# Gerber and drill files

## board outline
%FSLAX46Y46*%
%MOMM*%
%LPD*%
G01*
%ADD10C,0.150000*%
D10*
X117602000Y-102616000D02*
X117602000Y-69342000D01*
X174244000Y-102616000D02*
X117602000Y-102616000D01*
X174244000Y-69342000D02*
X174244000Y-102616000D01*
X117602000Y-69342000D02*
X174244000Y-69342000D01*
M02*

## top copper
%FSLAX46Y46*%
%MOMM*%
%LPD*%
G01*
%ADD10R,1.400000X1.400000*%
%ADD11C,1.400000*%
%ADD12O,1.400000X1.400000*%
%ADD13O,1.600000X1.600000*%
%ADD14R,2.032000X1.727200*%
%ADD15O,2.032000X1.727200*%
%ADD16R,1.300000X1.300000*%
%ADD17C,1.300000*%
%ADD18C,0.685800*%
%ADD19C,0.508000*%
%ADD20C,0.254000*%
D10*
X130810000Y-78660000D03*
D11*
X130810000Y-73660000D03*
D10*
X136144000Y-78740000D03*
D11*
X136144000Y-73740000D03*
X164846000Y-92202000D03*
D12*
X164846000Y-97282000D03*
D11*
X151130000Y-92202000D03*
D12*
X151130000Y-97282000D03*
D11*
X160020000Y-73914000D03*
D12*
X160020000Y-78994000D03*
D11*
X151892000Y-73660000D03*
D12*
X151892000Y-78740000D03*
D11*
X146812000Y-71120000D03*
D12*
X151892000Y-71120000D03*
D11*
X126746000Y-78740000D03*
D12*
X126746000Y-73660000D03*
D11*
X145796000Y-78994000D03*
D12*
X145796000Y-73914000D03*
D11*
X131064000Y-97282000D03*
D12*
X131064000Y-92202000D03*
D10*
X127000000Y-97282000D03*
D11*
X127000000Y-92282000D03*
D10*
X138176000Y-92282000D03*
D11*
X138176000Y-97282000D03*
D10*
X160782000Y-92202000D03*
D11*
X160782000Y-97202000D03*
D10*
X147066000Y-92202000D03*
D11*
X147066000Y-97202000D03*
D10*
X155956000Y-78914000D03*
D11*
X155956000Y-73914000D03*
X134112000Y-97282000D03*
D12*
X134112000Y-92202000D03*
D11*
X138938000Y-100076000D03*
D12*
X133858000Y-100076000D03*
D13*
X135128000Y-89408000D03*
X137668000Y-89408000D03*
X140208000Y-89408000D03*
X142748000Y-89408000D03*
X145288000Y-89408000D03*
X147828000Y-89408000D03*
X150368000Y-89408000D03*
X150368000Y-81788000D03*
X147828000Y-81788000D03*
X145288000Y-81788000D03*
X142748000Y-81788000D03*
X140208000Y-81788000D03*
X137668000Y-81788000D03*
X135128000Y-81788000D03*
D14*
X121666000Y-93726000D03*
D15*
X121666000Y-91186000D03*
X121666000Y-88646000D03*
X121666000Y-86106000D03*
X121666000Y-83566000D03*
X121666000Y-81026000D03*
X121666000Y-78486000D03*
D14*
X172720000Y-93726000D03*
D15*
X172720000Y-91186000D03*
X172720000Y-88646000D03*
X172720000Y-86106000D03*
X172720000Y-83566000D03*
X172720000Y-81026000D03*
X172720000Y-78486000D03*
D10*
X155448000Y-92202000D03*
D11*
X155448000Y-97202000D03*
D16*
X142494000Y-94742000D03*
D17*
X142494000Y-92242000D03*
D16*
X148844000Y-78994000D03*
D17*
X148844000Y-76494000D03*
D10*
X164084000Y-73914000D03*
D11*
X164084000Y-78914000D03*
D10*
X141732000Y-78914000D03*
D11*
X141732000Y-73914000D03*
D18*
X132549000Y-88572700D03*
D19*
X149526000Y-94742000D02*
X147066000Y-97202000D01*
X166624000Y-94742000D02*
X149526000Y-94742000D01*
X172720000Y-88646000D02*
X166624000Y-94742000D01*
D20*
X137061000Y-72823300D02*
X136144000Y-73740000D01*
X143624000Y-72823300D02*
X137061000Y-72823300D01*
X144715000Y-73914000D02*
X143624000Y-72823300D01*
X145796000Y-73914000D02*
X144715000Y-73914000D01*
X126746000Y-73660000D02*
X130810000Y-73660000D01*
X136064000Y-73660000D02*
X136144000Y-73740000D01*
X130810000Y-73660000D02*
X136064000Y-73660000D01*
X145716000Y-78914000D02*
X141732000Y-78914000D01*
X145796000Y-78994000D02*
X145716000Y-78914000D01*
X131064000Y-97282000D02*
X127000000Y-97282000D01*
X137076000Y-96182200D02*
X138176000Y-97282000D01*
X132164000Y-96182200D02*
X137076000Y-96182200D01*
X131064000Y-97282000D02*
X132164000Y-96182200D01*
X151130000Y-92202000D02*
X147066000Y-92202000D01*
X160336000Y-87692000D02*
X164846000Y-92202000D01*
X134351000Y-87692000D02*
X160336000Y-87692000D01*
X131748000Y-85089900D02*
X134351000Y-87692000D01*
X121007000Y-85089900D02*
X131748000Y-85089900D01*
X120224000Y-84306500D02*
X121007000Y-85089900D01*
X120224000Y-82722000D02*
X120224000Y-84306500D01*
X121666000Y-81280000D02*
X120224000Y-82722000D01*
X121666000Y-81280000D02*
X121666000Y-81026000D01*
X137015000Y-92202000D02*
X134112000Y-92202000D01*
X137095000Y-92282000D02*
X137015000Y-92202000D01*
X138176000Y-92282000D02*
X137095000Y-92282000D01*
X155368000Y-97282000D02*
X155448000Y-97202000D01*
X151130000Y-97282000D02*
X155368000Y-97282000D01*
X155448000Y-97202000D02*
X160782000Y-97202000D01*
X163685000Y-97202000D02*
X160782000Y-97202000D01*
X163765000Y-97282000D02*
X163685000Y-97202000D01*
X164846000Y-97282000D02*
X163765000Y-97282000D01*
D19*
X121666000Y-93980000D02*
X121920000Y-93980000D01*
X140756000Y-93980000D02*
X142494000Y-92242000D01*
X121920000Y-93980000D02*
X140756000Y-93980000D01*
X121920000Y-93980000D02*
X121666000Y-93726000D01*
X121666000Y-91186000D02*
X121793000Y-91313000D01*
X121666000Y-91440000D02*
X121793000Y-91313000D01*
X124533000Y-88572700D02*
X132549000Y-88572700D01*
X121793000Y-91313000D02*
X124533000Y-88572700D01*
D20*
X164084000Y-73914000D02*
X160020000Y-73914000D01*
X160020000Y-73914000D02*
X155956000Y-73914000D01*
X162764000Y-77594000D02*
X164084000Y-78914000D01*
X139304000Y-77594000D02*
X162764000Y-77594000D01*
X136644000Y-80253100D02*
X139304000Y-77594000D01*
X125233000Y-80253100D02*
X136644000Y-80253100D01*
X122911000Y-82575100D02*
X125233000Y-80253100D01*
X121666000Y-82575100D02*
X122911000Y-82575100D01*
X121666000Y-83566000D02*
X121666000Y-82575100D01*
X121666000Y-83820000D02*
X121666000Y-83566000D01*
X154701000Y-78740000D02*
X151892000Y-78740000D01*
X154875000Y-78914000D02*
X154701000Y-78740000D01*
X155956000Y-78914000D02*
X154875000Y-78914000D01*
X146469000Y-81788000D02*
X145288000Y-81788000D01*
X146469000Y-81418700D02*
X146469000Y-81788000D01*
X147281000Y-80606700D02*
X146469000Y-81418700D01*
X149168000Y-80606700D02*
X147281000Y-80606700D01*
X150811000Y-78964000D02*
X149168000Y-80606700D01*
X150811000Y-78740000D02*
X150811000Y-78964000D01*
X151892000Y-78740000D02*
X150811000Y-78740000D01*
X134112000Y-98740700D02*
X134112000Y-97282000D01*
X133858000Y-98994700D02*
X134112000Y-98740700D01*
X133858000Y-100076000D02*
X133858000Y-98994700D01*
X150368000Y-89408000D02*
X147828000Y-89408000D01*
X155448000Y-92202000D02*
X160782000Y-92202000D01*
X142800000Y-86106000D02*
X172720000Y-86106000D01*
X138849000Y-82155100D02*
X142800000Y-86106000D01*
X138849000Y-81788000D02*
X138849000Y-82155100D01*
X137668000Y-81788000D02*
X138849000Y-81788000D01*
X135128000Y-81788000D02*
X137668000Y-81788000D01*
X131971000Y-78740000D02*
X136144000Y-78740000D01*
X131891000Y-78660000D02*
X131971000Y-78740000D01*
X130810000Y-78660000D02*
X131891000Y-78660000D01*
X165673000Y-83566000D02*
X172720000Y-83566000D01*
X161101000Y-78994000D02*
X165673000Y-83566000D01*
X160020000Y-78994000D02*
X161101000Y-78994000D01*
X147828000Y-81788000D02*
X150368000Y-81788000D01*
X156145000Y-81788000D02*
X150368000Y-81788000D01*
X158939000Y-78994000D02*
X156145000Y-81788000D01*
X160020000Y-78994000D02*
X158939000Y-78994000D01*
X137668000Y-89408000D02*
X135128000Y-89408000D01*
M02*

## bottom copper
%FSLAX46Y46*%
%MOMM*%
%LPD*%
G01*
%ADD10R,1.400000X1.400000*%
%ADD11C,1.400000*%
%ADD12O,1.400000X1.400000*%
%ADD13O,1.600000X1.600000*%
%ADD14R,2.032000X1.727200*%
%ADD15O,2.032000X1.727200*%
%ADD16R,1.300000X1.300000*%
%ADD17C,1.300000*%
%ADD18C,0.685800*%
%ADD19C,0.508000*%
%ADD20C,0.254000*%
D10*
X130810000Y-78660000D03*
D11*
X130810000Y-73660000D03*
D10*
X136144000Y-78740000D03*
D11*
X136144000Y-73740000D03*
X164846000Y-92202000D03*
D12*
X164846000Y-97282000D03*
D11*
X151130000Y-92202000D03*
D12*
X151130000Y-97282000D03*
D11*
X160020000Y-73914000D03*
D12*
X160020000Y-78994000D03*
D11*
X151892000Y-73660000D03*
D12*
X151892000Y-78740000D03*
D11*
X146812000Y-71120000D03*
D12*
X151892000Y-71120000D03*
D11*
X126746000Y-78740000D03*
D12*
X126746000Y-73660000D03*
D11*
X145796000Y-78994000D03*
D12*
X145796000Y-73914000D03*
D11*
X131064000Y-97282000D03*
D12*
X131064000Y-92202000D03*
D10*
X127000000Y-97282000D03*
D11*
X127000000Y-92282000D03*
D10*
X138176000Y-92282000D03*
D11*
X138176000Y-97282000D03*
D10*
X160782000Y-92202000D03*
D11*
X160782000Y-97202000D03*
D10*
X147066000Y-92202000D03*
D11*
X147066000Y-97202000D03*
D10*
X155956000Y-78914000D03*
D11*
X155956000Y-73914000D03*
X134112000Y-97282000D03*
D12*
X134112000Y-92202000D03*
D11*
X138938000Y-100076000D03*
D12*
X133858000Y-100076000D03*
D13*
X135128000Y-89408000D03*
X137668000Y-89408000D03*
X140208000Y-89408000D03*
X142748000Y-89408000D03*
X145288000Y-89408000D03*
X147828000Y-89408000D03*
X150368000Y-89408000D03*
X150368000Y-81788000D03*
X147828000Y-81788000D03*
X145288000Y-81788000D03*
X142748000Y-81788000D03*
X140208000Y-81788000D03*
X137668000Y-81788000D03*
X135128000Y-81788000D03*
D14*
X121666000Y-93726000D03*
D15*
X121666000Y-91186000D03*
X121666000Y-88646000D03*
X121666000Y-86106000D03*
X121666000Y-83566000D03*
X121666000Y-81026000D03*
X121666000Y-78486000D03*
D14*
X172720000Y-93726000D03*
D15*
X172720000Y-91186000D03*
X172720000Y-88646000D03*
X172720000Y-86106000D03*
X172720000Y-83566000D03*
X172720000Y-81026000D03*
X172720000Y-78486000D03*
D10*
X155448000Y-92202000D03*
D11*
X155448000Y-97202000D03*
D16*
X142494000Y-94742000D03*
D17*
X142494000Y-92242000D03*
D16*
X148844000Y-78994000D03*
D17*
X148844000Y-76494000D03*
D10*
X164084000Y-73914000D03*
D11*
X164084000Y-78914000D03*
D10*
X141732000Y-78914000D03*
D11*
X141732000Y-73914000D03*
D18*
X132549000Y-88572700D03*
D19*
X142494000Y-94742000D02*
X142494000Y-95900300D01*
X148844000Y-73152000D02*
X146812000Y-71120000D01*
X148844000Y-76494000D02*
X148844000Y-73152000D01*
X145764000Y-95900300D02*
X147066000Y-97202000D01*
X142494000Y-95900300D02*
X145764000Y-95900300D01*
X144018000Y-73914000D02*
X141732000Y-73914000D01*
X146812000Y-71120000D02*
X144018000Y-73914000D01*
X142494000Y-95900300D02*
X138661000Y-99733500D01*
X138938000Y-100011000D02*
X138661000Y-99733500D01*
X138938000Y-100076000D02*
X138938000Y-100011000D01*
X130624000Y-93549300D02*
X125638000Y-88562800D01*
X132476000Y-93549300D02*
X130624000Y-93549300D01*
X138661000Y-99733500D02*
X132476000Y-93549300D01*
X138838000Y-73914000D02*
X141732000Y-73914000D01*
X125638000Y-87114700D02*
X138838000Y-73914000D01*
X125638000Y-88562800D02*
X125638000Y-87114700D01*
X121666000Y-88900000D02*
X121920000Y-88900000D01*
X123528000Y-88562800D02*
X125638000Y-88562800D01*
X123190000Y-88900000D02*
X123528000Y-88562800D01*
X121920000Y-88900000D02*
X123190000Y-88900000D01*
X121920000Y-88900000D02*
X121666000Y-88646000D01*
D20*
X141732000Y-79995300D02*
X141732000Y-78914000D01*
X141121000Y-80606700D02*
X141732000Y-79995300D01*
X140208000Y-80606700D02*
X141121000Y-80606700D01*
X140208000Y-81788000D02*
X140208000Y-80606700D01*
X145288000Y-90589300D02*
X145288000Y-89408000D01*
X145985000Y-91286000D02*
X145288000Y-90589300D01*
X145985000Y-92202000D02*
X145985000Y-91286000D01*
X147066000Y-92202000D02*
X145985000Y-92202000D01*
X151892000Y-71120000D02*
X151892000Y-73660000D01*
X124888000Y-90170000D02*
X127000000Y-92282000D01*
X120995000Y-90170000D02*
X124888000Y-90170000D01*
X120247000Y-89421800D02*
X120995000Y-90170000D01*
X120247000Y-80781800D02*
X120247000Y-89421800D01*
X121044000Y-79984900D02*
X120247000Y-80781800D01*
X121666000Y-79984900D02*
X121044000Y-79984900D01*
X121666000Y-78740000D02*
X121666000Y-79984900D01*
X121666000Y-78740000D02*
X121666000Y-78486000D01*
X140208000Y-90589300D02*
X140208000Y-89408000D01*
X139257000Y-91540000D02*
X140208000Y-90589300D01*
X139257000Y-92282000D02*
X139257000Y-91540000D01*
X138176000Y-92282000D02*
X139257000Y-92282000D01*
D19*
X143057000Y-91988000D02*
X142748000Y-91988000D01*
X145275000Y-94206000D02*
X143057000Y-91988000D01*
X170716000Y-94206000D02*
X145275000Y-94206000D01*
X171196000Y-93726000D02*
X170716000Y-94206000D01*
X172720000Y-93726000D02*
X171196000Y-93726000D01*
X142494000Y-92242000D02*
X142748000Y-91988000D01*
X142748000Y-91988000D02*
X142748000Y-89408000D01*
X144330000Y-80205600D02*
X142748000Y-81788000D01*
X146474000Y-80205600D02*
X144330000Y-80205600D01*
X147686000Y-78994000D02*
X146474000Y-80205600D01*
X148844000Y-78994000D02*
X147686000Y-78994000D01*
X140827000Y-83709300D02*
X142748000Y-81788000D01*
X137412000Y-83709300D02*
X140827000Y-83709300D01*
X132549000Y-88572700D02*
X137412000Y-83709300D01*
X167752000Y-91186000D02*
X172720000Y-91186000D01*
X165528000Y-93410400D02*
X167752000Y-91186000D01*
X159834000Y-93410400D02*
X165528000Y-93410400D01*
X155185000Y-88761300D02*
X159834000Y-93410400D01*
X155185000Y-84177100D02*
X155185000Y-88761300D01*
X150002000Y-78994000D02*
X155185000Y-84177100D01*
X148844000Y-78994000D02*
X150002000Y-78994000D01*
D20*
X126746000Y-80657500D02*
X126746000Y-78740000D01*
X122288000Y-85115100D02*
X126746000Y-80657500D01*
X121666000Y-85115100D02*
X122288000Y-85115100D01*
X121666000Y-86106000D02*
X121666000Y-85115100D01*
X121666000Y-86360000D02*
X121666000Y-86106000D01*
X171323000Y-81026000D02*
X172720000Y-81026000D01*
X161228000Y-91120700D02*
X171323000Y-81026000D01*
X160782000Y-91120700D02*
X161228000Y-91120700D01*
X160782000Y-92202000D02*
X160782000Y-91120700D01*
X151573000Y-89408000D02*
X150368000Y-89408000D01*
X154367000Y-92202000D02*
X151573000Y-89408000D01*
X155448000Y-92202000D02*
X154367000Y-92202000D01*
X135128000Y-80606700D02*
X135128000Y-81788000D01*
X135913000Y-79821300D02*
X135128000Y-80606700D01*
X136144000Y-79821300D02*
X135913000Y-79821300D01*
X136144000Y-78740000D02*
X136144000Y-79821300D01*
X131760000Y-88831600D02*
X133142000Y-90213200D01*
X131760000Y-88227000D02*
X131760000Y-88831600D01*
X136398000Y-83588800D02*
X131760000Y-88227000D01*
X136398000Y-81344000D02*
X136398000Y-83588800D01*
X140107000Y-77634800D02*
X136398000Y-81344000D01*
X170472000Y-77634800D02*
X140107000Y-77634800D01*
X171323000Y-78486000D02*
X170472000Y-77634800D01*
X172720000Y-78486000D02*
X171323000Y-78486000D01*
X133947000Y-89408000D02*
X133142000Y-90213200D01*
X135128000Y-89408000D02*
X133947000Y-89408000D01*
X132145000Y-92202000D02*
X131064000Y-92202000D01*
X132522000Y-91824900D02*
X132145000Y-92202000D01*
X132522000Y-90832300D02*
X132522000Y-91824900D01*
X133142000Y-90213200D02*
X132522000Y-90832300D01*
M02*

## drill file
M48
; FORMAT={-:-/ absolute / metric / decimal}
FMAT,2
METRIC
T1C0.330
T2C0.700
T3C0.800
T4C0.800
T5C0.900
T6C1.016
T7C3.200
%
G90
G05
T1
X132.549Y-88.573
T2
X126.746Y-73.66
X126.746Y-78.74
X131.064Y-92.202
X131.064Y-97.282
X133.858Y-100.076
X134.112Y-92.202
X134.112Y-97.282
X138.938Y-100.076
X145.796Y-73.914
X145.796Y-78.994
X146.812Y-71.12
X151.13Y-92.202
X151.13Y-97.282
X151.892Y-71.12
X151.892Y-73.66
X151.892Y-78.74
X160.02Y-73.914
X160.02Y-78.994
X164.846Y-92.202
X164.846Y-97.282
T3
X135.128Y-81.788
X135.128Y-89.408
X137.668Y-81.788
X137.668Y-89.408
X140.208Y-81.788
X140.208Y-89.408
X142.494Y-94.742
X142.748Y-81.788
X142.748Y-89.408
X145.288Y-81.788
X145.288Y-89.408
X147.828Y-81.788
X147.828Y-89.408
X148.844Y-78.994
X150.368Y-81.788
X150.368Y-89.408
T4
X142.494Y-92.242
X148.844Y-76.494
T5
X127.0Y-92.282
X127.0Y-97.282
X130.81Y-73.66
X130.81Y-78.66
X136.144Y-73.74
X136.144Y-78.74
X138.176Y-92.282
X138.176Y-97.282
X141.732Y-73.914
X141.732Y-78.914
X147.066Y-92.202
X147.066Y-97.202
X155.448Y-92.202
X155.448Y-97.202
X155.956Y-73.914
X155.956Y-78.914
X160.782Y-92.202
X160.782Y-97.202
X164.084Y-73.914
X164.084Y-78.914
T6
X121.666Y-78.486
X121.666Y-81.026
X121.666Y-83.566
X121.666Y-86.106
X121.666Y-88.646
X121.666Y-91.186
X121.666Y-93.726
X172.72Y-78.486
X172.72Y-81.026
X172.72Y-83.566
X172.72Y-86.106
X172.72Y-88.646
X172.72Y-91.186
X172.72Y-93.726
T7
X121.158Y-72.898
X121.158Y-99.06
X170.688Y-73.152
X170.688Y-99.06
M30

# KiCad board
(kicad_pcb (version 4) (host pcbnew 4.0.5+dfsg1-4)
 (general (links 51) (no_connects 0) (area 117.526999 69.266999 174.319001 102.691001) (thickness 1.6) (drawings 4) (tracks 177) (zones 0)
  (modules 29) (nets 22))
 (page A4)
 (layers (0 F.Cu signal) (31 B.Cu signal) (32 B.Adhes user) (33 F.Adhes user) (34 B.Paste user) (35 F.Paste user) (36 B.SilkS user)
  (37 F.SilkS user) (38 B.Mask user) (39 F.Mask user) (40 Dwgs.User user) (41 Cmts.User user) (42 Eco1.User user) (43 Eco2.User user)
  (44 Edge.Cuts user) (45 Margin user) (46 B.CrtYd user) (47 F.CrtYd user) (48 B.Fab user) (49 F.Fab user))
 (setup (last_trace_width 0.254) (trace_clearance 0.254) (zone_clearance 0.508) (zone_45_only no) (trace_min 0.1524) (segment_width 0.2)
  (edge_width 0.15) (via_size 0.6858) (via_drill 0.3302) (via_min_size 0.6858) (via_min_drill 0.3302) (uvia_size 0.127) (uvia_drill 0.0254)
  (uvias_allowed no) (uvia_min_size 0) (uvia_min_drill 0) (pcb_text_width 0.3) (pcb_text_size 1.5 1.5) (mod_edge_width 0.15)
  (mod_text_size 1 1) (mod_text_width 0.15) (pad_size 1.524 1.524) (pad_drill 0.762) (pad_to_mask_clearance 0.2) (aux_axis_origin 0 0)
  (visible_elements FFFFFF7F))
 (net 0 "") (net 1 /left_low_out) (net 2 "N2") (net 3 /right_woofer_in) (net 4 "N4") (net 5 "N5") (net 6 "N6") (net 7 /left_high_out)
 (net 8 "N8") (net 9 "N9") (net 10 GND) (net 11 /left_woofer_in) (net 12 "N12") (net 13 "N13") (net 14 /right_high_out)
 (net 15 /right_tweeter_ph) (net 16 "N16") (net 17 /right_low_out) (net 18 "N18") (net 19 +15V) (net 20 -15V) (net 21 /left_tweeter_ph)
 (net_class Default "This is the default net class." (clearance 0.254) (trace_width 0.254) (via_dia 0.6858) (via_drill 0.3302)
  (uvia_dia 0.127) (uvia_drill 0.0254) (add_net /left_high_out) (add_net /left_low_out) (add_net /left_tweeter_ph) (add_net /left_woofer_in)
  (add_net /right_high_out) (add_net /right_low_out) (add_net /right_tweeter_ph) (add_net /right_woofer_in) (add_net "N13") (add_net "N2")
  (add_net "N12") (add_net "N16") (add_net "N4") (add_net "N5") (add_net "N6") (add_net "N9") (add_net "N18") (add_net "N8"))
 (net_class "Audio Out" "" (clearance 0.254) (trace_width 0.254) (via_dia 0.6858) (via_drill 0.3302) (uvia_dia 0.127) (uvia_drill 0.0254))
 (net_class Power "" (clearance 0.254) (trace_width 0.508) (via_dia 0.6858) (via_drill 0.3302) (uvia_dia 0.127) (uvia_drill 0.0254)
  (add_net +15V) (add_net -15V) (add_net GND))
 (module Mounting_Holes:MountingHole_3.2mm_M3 (layer F.Cu) (at 121.158 99.06)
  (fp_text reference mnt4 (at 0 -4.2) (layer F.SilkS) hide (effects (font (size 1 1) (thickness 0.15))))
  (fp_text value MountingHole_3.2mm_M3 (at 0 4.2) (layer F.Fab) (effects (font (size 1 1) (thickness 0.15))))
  (pad 1 np_thru_hole circle (at 0 0) (size 3.2 3.2) (drill 3.2) (layers *.Cu *.Mask)))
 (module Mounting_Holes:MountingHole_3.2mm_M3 (layer F.Cu) (at 121.158 72.898)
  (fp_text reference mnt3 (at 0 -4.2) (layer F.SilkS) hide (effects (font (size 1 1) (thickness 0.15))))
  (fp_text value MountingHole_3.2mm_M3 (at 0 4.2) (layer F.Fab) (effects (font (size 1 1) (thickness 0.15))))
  (pad 1 np_thru_hole circle (at 0 0) (size 3.2 3.2) (drill 3.2) (layers *.Cu *.Mask)))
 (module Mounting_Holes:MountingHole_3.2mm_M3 (layer F.Cu) (at 170.688 99.06)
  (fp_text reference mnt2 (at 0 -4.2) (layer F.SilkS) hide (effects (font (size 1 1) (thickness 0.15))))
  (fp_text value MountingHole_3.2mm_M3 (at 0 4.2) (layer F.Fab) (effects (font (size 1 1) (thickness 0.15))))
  (pad 1 np_thru_hole circle (at 0 0) (size 3.2 3.2) (drill 3.2) (layers *.Cu *.Mask)))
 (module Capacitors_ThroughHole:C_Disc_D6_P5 (layer F.Cu) (at 130.81 78.66 90)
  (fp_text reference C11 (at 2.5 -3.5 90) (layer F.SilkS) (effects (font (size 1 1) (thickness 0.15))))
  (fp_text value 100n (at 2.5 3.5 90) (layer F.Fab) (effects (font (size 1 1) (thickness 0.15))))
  (pad 1 thru_hole rect (at 0 0 90) (size 1.4 1.4) (drill 0.9) (layers *.Cu *.Mask) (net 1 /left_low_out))
  (pad 2 thru_hole circle (at 5 0 90) (size 1.4 1.4) (drill 0.9) (layers *.Cu *.Mask) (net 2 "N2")))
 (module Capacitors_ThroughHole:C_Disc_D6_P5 (layer F.Cu) (at 136.144 78.74 90)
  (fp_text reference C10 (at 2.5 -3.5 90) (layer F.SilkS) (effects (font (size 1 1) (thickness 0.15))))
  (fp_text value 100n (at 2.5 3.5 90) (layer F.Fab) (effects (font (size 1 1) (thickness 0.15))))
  (pad 1 thru_hole rect (at 0 0 90) (size 1.4 1.4) (drill 0.9) (layers *.Cu *.Mask) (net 1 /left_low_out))
  (pad 2 thru_hole circle (at 5 0 90) (size 1.4 1.4) (drill 0.9) (layers *.Cu *.Mask) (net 2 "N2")))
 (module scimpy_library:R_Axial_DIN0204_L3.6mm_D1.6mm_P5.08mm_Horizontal (layer F.Cu) (at 164.846 92.202 270)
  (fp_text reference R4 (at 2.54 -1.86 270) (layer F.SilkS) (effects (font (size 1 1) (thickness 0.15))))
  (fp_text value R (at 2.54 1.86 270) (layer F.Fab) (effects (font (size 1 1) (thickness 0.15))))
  (pad 1 thru_hole circle (at 0 0 270) (size 1.4 1.4) (drill 0.7) (layers *.Cu *.Mask) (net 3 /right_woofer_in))
  (pad 2 thru_hole oval (at 5.08 0 270) (size 1.4 1.4) (drill 0.7) (layers *.Cu *.Mask) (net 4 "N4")))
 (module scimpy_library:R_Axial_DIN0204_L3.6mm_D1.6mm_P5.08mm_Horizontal (layer F.Cu) (at 151.13 92.202 270)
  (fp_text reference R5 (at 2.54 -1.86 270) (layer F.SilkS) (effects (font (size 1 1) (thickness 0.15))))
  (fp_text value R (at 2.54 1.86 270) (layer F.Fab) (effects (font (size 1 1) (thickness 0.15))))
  (pad 1 thru_hole circle (at 0 0 270) (size 1.4 1.4) (drill 0.7) (layers *.Cu *.Mask) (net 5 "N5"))
  (pad 2 thru_hole oval (at 5.08 0 270) (size 1.4 1.4) (drill 0.7) (layers *.Cu *.Mask) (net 4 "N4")))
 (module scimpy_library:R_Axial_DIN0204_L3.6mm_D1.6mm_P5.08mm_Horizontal (layer F.Cu) (at 160.02 73.914 270)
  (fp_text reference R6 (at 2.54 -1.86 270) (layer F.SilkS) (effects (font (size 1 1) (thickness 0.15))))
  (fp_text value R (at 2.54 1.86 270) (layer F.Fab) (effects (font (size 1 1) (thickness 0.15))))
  (pad 1 thru_hole circle (at 0 0 270) (size 1.4 1.4) (drill 0.7) (layers *.Cu *.Mask) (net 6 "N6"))
  (pad 2 thru_hole oval (at 5.08 0 270) (size 1.4 1.4) (drill 0.7) (layers *.Cu *.Mask) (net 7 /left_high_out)))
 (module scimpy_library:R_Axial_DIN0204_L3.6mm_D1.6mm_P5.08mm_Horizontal (layer F.Cu) (at 151.892 73.66 270)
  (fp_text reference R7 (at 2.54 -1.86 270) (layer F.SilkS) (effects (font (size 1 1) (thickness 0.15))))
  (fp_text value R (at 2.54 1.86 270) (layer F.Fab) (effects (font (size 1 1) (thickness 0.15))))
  (pad 1 thru_hole circle (at 0 0 270) (size 1.4 1.4) (drill 0.7) (layers *.Cu *.Mask) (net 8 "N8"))
  (pad 2 thru_hole oval (at 5.08 0 270) (size 1.4 1.4) (drill 0.7) (layers *.Cu *.Mask) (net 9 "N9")))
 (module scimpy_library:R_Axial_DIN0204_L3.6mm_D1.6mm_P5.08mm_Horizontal (layer F.Cu) (at 146.812 71.12)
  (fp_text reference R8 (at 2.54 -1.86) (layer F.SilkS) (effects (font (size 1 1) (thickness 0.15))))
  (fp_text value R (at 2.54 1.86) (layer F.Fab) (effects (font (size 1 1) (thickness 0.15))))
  (pad 1 thru_hole circle (at 0 0) (size 1.4 1.4) (drill 0.7) (layers *.Cu *.Mask) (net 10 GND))
  (pad 2 thru_hole oval (at 5.08 0) (size 1.4 1.4) (drill 0.7) (layers *.Cu *.Mask) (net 8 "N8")))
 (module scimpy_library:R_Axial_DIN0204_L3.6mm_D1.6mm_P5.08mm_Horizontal (layer F.Cu) (at 126.746 78.74 90)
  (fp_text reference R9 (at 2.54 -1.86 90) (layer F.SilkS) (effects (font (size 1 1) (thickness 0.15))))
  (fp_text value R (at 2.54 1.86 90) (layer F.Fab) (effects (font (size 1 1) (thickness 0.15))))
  (pad 1 thru_hole circle (at 0 0 90) (size 1.4 1.4) (drill 0.7) (layers *.Cu *.Mask) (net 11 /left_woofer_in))
  (pad 2 thru_hole oval (at 5.08 0 90) (size 1.4 1.4) (drill 0.7) (layers *.Cu *.Mask) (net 2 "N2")))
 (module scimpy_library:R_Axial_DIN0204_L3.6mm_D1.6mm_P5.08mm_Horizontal (layer F.Cu) (at 145.796 78.994 90)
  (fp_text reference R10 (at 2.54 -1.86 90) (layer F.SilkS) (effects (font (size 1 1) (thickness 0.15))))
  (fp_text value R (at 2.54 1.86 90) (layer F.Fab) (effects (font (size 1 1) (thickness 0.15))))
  (pad 1 thru_hole circle (at 0 0 90) (size 1.4 1.4) (drill 0.7) (layers *.Cu *.Mask) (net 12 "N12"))
  (pad 2 thru_hole oval (at 5.08 0 90) (size 1.4 1.4) (drill 0.7) (layers *.Cu *.Mask) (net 2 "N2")))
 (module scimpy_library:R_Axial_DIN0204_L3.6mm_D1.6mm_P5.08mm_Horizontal (layer F.Cu) (at 131.064 97.282 90)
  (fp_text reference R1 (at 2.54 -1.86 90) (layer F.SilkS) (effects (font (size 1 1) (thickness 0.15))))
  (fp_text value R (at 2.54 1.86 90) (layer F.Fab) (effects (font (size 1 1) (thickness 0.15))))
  (pad 1 thru_hole circle (at 0 0 90) (size 1.4 1.4) (drill 0.7) (layers *.Cu *.Mask) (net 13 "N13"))
  (pad 2 thru_hole oval (at 5.08 0 90) (size 1.4 1.4) (drill 0.7) (layers *.Cu *.Mask) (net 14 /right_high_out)))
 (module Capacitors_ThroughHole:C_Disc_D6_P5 (layer F.Cu) (at 127 97.282 90)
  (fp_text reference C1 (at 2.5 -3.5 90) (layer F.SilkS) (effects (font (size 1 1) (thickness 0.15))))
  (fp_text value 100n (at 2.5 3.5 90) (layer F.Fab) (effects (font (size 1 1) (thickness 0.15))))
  (pad 1 thru_hole rect (at 0 0 90) (size 1.4 1.4) (drill 0.9) (layers *.Cu *.Mask) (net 13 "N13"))
  (pad 2 thru_hole circle (at 5 0 90) (size 1.4 1.4) (drill 0.9) (layers *.Cu *.Mask) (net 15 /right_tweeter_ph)))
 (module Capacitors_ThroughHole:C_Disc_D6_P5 (layer F.Cu) (at 138.176 92.282 270)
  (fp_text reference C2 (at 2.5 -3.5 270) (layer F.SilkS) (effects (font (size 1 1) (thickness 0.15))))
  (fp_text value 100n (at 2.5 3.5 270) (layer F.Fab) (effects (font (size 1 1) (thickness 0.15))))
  (pad 1 thru_hole rect (at 0 0 270) (size 1.4 1.4) (drill 0.9) (layers *.Cu *.Mask) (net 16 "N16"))
  (pad 2 thru_hole circle (at 5 0 270) (size 1.4 1.4) (drill 0.9) (layers *.Cu *.Mask) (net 13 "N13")))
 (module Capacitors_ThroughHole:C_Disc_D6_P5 (layer F.Cu) (at 160.782 92.202 270)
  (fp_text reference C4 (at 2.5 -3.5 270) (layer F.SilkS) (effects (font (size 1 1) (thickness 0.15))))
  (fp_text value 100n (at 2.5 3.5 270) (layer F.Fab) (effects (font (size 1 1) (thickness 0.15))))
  (pad 1 thru_hole rect (at 0 0 270) (size 1.4 1.4) (drill 0.9) (layers *.Cu *.Mask) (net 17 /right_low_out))
  (pad 2 thru_hole circle (at 5 0 270) (size 1.4 1.4) (drill 0.9) (layers *.Cu *.Mask) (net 4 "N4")))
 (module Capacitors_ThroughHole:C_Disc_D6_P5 (layer F.Cu) (at 147.066 92.202 270)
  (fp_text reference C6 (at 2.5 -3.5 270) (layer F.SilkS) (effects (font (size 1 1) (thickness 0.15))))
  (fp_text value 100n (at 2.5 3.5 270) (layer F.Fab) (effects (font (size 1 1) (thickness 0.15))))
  (pad 1 thru_hole rect (at 0 0 270) (size 1.4 1.4) (drill 0.9) (layers *.Cu *.Mask) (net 5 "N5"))
  (pad 2 thru_hole circle (at 5 0 270) (size 1.4 1.4) (drill 0.9) (layers *.Cu *.Mask) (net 10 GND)))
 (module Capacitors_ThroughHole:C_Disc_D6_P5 (layer F.Cu) (at 155.956 78.914 90)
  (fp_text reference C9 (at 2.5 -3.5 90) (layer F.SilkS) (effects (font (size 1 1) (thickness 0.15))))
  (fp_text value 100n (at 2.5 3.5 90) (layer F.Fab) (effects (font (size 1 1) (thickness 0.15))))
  (pad 1 thru_hole rect (at 0 0 90) (size 1.4 1.4) (drill 0.9) (layers *.Cu *.Mask) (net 9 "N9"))
  (pad 2 thru_hole circle (at 5 0 90) (size 1.4 1.4) (drill 0.9) (layers *.Cu *.Mask) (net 6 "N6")))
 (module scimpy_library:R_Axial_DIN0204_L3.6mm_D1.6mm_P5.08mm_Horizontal (layer F.Cu) (at 134.112 97.282 90)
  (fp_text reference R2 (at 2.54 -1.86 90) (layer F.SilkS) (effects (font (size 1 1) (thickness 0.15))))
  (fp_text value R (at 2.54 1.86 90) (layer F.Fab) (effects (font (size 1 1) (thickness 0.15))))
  (pad 1 thru_hole circle (at 0 0 90) (size 1.4 1.4) (drill 0.7) (layers *.Cu *.Mask) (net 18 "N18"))
  (pad 2 thru_hole oval (at 5.08 0 90) (size 1.4 1.4) (drill 0.7) (layers *.Cu *.Mask) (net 16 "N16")))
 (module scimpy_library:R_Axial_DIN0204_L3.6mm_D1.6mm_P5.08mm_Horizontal (layer F.Cu) (at 138.938 100.076 180)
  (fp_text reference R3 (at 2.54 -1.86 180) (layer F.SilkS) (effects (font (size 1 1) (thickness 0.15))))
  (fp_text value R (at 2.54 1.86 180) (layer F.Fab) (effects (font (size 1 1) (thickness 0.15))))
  (pad 1 thru_hole circle (at 0 0 180) (size 1.4 1.4) (drill 0.7) (layers *.Cu *.Mask) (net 10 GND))
  (pad 2 thru_hole oval (at 5.08 0 180) (size 1.4 1.4) (drill 0.7) (layers *.Cu *.Mask) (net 18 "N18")))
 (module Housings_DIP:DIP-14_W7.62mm (layer F.Cu) (at 135.128 89.408 90)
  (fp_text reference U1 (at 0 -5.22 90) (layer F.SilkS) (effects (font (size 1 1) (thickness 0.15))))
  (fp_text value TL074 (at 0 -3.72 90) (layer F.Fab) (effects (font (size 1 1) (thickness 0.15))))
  (pad 1 thru_hole oval (at 0 0 90) (size 1.6 1.6) (drill 0.8) (layers *.Cu *.Mask) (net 14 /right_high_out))
  (pad 2 thru_hole oval (at 0 2.54 90) (size 1.6 1.6) (drill 0.8) (layers *.Cu *.Mask) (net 14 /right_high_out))
  (pad 3 thru_hole oval (at 0 5.08 90) (size 1.6 1.6) (drill 0.8) (layers *.Cu *.Mask) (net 16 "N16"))
  (pad 4 thru_hole oval (at 0 7.62 90) (size 1.6 1.6) (drill 0.8) (layers *.Cu *.Mask) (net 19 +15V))
  (pad 5 thru_hole oval (at 0 10.16 90) (size 1.6 1.6) (drill 0.8) (layers *.Cu *.Mask) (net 5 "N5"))
  (pad 6 thru_hole oval (at 0 12.7 90) (size 1.6 1.6) (drill 0.8) (layers *.Cu *.Mask) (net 17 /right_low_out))
  (pad 7 thru_hole oval (at 0 15.24 90) (size 1.6 1.6) (drill 0.8) (layers *.Cu *.Mask) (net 17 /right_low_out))
  (pad 8 thru_hole oval (at 7.62 15.24 90) (size 1.6 1.6) (drill 0.8) (layers *.Cu *.Mask) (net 7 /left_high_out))
  (pad 9 thru_hole oval (at 7.62 12.7 90) (size 1.6 1.6) (drill 0.8) (layers *.Cu *.Mask) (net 7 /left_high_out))
  (pad 10 thru_hole oval (at 7.62 10.16 90) (size 1.6 1.6) (drill 0.8) (layers *.Cu *.Mask) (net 9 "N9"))
  (pad 11 thru_hole oval (at 7.62 7.62 90) (size 1.6 1.6) (drill 0.8) (layers *.Cu *.Mask) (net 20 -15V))
  (pad 12 thru_hole oval (at 7.62 5.08 90) (size 1.6 1.6) (drill 0.8) (layers *.Cu *.Mask) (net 12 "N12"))
  (pad 13 thru_hole oval (at 7.62 2.54 90) (size 1.6 1.6) (drill 0.8) (layers *.Cu *.Mask) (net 1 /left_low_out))
  (pad 14 thru_hole oval (at 7.62 0 90) (size 1.6 1.6) (drill 0.8) (layers *.Cu *.Mask) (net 1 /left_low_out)))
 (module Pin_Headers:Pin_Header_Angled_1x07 (layer F.Cu) (at 121.666 93.726 180)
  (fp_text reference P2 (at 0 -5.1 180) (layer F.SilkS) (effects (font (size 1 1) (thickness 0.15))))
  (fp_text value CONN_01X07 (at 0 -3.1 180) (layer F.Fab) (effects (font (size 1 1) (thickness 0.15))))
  (pad 1 thru_hole rect (at 0 0 180) (size 2.032 1.7272) (drill 1.016) (layers *.Cu *.Mask) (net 19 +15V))
  (pad 2 thru_hole oval (at 0 2.54 180) (size 2.032 1.7272) (drill 1.016) (layers *.Cu *.Mask) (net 20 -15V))
  (pad 3 thru_hole oval (at 0 5.08 180) (size 2.032 1.7272) (drill 1.016) (layers *.Cu *.Mask) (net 10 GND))
  (pad 4 thru_hole oval (at 0 7.62 180) (size 2.032 1.7272) (drill 1.016) (layers *.Cu *.Mask) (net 11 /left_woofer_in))
  (pad 5 thru_hole oval (at 0 10.16 180) (size 2.032 1.7272) (drill 1.016) (layers *.Cu *.Mask) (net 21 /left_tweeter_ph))
  (pad 6 thru_hole oval (at 0 12.7 180) (size 2.032 1.7272) (drill 1.016) (layers *.Cu *.Mask) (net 3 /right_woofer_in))
  (pad 7 thru_hole oval (at 0 15.24 180) (size 2.032 1.7272) (drill 1.016) (layers *.Cu *.Mask) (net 15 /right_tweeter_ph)))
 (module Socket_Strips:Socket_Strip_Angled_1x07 (layer F.Cu) (at 172.72 93.726 90)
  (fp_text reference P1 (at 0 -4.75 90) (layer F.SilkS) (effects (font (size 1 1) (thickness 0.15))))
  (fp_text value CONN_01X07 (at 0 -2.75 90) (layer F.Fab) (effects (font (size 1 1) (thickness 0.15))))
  (pad 1 thru_hole rect (at 0 0 90) (size 1.7272 2.032) (drill 1.016) (layers *.Cu *.Mask) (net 19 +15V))
  (pad 2 thru_hole oval (at 2.54 0 90) (size 1.7272 2.032) (drill 1.016) (layers *.Cu *.Mask) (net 20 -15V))
  (pad 3 thru_hole oval (at 5.08 0 90) (size 1.7272 2.032) (drill 1.016) (layers *.Cu *.Mask) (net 10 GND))
  (pad 4 thru_hole oval (at 7.62 0 90) (size 1.7272 2.032) (drill 1.016) (layers *.Cu *.Mask) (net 1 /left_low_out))
  (pad 5 thru_hole oval (at 10.16 0 90) (size 1.7272 2.032) (drill 1.016) (layers *.Cu *.Mask) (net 7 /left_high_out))
  (pad 6 thru_hole oval (at 12.7 0 90) (size 1.7272 2.032) (drill 1.016) (layers *.Cu *.Mask) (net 17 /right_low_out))
  (pad 7 thru_hole oval (at 15.24 0 90) (size 1.7272 2.032) (drill 1.016) (layers *.Cu *.Mask) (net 14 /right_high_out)))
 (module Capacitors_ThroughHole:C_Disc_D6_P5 (layer F.Cu) (at 155.448 92.202 270)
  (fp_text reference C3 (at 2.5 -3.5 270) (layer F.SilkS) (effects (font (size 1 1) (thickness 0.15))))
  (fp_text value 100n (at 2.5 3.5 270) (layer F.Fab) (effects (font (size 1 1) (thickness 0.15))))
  (pad 1 thru_hole rect (at 0 0 270) (size 1.4 1.4) (drill 0.9) (layers *.Cu *.Mask) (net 17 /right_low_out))
  (pad 2 thru_hole circle (at 5 0 270) (size 1.4 1.4) (drill 0.9) (layers *.Cu *.Mask) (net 4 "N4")))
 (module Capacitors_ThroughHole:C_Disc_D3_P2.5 (layer F.Cu) (at 142.494 94.742 90)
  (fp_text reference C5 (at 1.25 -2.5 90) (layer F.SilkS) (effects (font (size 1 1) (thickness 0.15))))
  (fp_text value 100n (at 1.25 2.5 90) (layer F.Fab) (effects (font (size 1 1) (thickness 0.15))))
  (pad 1 thru_hole rect (at 0 0 90) (size 1.3 1.3) (drill 0.8) (layers *.Cu *.Mask) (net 10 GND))
  (pad 2 thru_hole circle (at 2.5 0 90) (size 1.3 1.3) (drill 0.8001) (layers *.Cu *.Mask) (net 19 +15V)))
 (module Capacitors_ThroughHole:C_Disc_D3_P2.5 (layer F.Cu) (at 148.844 78.994 90)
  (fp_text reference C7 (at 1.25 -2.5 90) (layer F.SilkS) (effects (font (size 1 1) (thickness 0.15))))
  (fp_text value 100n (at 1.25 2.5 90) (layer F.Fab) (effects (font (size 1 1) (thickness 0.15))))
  (pad 1 thru_hole rect (at 0 0 90) (size 1.3 1.3) (drill 0.8) (layers *.Cu *.Mask) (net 20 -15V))
  (pad 2 thru_hole circle (at 2.5 0 90) (size 1.3 1.3) (drill 0.8001) (layers *.Cu *.Mask) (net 10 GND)))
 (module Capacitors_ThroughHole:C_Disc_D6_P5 (layer F.Cu) (at 164.084 73.914 270)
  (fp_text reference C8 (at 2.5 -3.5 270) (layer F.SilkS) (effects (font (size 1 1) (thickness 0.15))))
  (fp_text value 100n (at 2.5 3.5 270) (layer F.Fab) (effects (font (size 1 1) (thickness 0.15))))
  (pad 1 thru_hole rect (at 0 0 270) (size 1.4 1.4) (drill 0.9) (layers *.Cu *.Mask) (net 6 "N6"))
  (pad 2 thru_hole circle (at 5 0 270) (size 1.4 1.4) (drill 0.9) (layers *.Cu *.Mask) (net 21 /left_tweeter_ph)))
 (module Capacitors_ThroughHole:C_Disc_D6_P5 (layer F.Cu) (at 141.732 78.914 90)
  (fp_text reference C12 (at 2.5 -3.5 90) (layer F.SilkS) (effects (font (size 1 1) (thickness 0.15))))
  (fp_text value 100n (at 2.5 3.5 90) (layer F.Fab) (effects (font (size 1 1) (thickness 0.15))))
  (pad 1 thru_hole rect (at 0 0 90) (size 1.4 1.4) (drill 0.9) (layers *.Cu *.Mask) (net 12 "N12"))
  (pad 2 thru_hole circle (at 5 0 90) (size 1.4 1.4) (drill 0.9) (layers *.Cu *.Mask) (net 10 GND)))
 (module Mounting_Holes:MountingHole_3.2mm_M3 (layer F.Cu) (at 170.688 73.152)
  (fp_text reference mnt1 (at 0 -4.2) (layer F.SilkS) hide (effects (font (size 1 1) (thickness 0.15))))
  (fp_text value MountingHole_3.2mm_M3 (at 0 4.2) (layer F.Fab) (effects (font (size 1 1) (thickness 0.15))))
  (pad 1 np_thru_hole circle (at 0 0) (size 3.2 3.2) (drill 3.2) (layers *.Cu *.Mask)))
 (gr_line (start 117.602 102.616) (end 117.602 69.342) (angle 90) (layer Edge.Cuts) (width 0.15))
 (gr_line (start 174.244 102.616) (end 117.602 102.616) (angle 90) (layer Edge.Cuts) (width 0.15))
 (gr_line (start 174.244 69.342) (end 174.244 102.616) (angle 90) (layer Edge.Cuts) (width 0.15))
 (gr_line (start 117.602 69.342) (end 174.244 69.342) (angle 90) (layer Edge.Cuts) (width 0.15))
 (segment (start 149.526 94.742) (end 147.066 97.202) (width 0.508) (layer F.Cu) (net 10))
 (segment (start 166.624 94.742) (end 149.526 94.742) (width 0.508) (layer F.Cu) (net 10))
 (segment (start 172.72 88.646) (end 166.624 94.742) (width 0.508) (layer F.Cu) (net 10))
 (segment (start 142.494 94.742) (end 142.494 95.9003) (width 0.508) (layer B.Cu) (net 10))
 (segment (start 148.844 73.152) (end 146.812 71.12) (width 0.508) (layer B.Cu) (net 10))
 (segment (start 148.844 76.494) (end 148.844 73.152) (width 0.508) (layer B.Cu) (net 10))
 (segment (start 145.764 95.9003) (end 147.066 97.202) (width 0.508) (layer B.Cu) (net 10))
 (segment (start 142.494 95.9003) (end 145.764 95.9003) (width 0.508) (layer B.Cu) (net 10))
 (segment (start 144.018 73.914) (end 141.732 73.914) (width 0.508) (layer B.Cu) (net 10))
 (segment (start 146.812 71.12) (end 144.018 73.914) (width 0.508) (layer B.Cu) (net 10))
 (segment (start 142.494 95.9003) (end 138.661 99.7335) (width 0.508) (layer B.Cu) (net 10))
 (segment (start 138.938 100.011) (end 138.661 99.7335) (width 0.508) (layer B.Cu) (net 10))
 (segment (start 138.938 100.076) (end 138.938 100.011) (width 0.508) (layer B.Cu) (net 10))
 (segment (start 130.624 93.5493) (end 125.638 88.5628) (width 0.508) (layer B.Cu) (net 10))
 (segment (start 132.476 93.5493) (end 130.624 93.5493) (width 0.508) (layer B.Cu) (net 10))
 (segment (start 138.661 99.7335) (end 132.476 93.5493) (width 0.508) (layer B.Cu) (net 10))
 (segment (start 138.838 73.914) (end 141.732 73.914) (width 0.508) (layer B.Cu) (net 10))
 (segment (start 125.638 87.1147) (end 138.838 73.914) (width 0.508) (layer B.Cu) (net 10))
 (segment (start 125.638 88.5628) (end 125.638 87.1147) (width 0.508) (layer B.Cu) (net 10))
 (segment (start 121.666 88.9) (end 121.92 88.9) (width 0.508) (layer B.Cu) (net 10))
 (segment (start 123.528 88.5628) (end 125.638 88.5628) (width 0.508) (layer B.Cu) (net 10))
 (segment (start 123.19 88.9) (end 123.528 88.5628) (width 0.508) (layer B.Cu) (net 10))
 (segment (start 121.92 88.9) (end 123.19 88.9) (width 0.508) (layer B.Cu) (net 10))
 (segment (start 121.92 88.9) (end 121.666 88.646) (width 0.508) (layer B.Cu) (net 10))
 (segment (start 137.061 72.8233) (end 136.144 73.74) (width 0.254) (layer F.Cu) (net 2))
 (segment (start 143.624 72.8233) (end 137.061 72.8233) (width 0.254) (layer F.Cu) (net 2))
 (segment (start 144.715 73.914) (end 143.624 72.8233) (width 0.254) (layer F.Cu) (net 2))
 (segment (start 145.796 73.914) (end 144.715 73.914) (width 0.254) (layer F.Cu) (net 2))
 (segment (start 126.746 73.66) (end 130.81 73.66) (width 0.254) (layer F.Cu) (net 2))
 (segment (start 136.064 73.66) (end 136.144 73.74) (width 0.254) (layer F.Cu) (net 2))
 (segment (start 130.81 73.66) (end 136.064 73.66) (width 0.254) (layer F.Cu) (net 2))
 (segment (start 141.732 79.9953) (end 141.732 78.914) (width 0.254) (layer B.Cu) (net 12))
 (segment (start 141.121 80.6067) (end 141.732 79.9953) (width 0.254) (layer B.Cu) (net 12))
 (segment (start 140.208 80.6067) (end 141.121 80.6067) (width 0.254) (layer B.Cu) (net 12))
 (segment (start 140.208 81.788) (end 140.208 80.6067) (width 0.254) (layer B.Cu) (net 12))
 (segment (start 145.716 78.914) (end 141.732 78.914) (width 0.254) (layer F.Cu) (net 12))
 (segment (start 145.796 78.994) (end 145.716 78.914) (width 0.254) (layer F.Cu) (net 12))
 (segment (start 131.064 97.282) (end 127 97.282) (width 0.254) (layer F.Cu) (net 13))
 (segment (start 137.076 96.1822) (end 138.176 97.282) (width 0.254) (layer F.Cu) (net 13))
 (segment (start 132.164 96.1822) (end 137.076 96.1822) (width 0.254) (layer F.Cu) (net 13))
 (segment (start 131.064 97.282) (end 132.164 96.1822) (width 0.254) (layer F.Cu) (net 13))
 (segment (start 151.13 92.202) (end 147.066 92.202) (width 0.254) (layer F.Cu) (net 5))
 (segment (start 145.288 90.5893) (end 145.288 89.408) (width 0.254) (layer B.Cu) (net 5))
 (segment (start 145.985 91.286) (end 145.288 90.5893) (width 0.254) (layer B.Cu) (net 5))
 (segment (start 145.985 92.202) (end 145.985 91.286) (width 0.254) (layer B.Cu) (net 5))
 (segment (start 147.066 92.202) (end 145.985 92.202) (width 0.254) (layer B.Cu) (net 5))
 (segment (start 151.892 71.12) (end 151.892 73.66) (width 0.254) (layer B.Cu) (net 8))
 (segment (start 124.888 90.17) (end 127 92.282) (width 0.254) (layer B.Cu) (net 15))
 (segment (start 120.995 90.17) (end 124.888 90.17) (width 0.254) (layer B.Cu) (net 15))
 (segment (start 120.247 89.4218) (end 120.995 90.17) (width 0.254) (layer B.Cu) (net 15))
 (segment (start 120.247 80.7818) (end 120.247 89.4218) (width 0.254) (layer B.Cu) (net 15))
 (segment (start 121.044 79.9849) (end 120.247 80.7818) (width 0.254) (layer B.Cu) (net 15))
 (segment (start 121.666 79.9849) (end 121.044 79.9849) (width 0.254) (layer B.Cu) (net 15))
 (segment (start 121.666 78.74) (end 121.666 79.9849) (width 0.254) (layer B.Cu) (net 15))
 (segment (start 121.666 78.74) (end 121.666 78.486) (width 0.254) (layer B.Cu) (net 15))
 (segment (start 160.336 87.692) (end 164.846 92.202) (width 0.254) (layer F.Cu) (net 3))
 (segment (start 134.351 87.692) (end 160.336 87.692) (width 0.254) (layer F.Cu) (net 3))
 (segment (start 131.748 85.0899) (end 134.351 87.692) (width 0.254) (layer F.Cu) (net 3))
 (segment (start 121.007 85.0899) (end 131.748 85.0899) (width 0.254) (layer F.Cu) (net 3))
 (segment (start 120.224 84.3065) (end 121.007 85.0899) (width 0.254) (layer F.Cu) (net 3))
 (segment (start 120.224 82.722) (end 120.224 84.3065) (width 0.254) (layer F.Cu) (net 3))
 (segment (start 121.666 81.28) (end 120.224 82.722) (width 0.254) (layer F.Cu) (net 3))
 (segment (start 121.666 81.28) (end 121.666 81.026) (width 0.254) (layer F.Cu) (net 3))
 (segment (start 140.208 90.5893) (end 140.208 89.408) (width 0.254) (layer B.Cu) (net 16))
 (segment (start 139.257 91.54) (end 140.208 90.5893) (width 0.254) (layer B.Cu) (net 16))
 (segment (start 139.257 92.282) (end 139.257 91.54) (width 0.254) (layer B.Cu) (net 16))
 (segment (start 138.176 92.282) (end 139.257 92.282) (width 0.254) (layer B.Cu) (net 16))
 (segment (start 137.015 92.202) (end 134.112 92.202) (width 0.254) (layer F.Cu) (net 16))
 (segment (start 137.095 92.282) (end 137.015 92.202) (width 0.254) (layer F.Cu) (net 16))
 (segment (start 138.176 92.282) (end 137.095 92.282) (width 0.254) (layer F.Cu) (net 16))
 (segment (start 155.368 97.282) (end 155.448 97.202) (width 0.254) (layer F.Cu) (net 4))
 (segment (start 151.13 97.282) (end 155.368 97.282) (width 0.254) (layer F.Cu) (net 4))
 (segment (start 155.448 97.202) (end 160.782 97.202) (width 0.254) (layer F.Cu) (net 4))
 (segment (start 163.685 97.202) (end 160.782 97.202) (width 0.254) (layer F.Cu) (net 4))
 (segment (start 163.765 97.282) (end 163.685 97.202) (width 0.254) (layer F.Cu) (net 4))
 (segment (start 164.846 97.282) (end 163.765 97.282) (width 0.254) (layer F.Cu) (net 4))
 (segment (start 143.057 91.988) (end 142.748 91.988) (width 0.508) (layer B.Cu) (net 19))
 (segment (start 145.275 94.206) (end 143.057 91.988) (width 0.508) (layer B.Cu) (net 19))
 (segment (start 170.716 94.206) (end 145.275 94.206) (width 0.508) (layer B.Cu) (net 19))
 (segment (start 171.196 93.726) (end 170.716 94.206) (width 0.508) (layer B.Cu) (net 19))
 (segment (start 172.72 93.726) (end 171.196 93.726) (width 0.508) (layer B.Cu) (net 19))
 (segment (start 142.494 92.242) (end 142.748 91.988) (width 0.508) (layer B.Cu) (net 19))
 (segment (start 142.748 91.988) (end 142.748 89.408) (width 0.508) (layer B.Cu) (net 19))
 (segment (start 121.666 93.98) (end 121.92 93.98) (width 0.508) (layer F.Cu) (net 19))
 (segment (start 140.756 93.98) (end 142.494 92.242) (width 0.508) (layer F.Cu) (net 19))
 (segment (start 121.92 93.98) (end 140.756 93.98) (width 0.508) (layer F.Cu) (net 19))
 (segment (start 121.92 93.98) (end 121.666 93.726) (width 0.508) (layer F.Cu) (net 19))
 (via (at 132.549 88.5727) (size 0.6858) (layers F.Cu B.Cu) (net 20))
 (segment (start 144.33 80.2056) (end 142.748 81.788) (width 0.508) (layer B.Cu) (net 20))
 (segment (start 146.474 80.2056) (end 144.33 80.2056) (width 0.508) (layer B.Cu) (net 20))
 (segment (start 147.686 78.994) (end 146.474 80.2056) (width 0.508) (layer B.Cu) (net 20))
 (segment (start 148.844 78.994) (end 147.686 78.994) (width 0.508) (layer B.Cu) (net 20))
 (segment (start 140.827 83.7093) (end 142.748 81.788) (width 0.508) (layer B.Cu) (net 20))
 (segment (start 137.412 83.7093) (end 140.827 83.7093) (width 0.508) (layer B.Cu) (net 20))
 (segment (start 132.549 88.5727) (end 137.412 83.7093) (width 0.508) (layer B.Cu) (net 20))
 (segment (start 167.752 91.186) (end 172.72 91.186) (width 0.508) (layer B.Cu) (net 20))
 (segment (start 165.528 93.4104) (end 167.752 91.186) (width 0.508) (layer B.Cu) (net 20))
 (segment (start 159.834 93.4104) (end 165.528 93.4104) (width 0.508) (layer B.Cu) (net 20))
 (segment (start 155.185 88.7613) (end 159.834 93.4104) (width 0.508) (layer B.Cu) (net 20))
 (segment (start 155.185 84.1771) (end 155.185 88.7613) (width 0.508) (layer B.Cu) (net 20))
 (segment (start 150.002 78.994) (end 155.185 84.1771) (width 0.508) (layer B.Cu) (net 20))
 (segment (start 148.844 78.994) (end 150.002 78.994) (width 0.508) (layer B.Cu) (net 20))
 (segment (start 121.666 91.186) (end 121.793 91.313) (width 0.508) (layer F.Cu) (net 20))
 (segment (start 121.666 91.44) (end 121.793 91.313) (width 0.508) (layer F.Cu) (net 20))
 (segment (start 124.533 88.5727) (end 132.549 88.5727) (width 0.508) (layer F.Cu) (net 20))
 (segment (start 121.793 91.313) (end 124.533 88.5727) (width 0.508) (layer F.Cu) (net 20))
 (segment (start 164.084 73.914) (end 160.02 73.914) (width 0.254) (layer F.Cu) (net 6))
 (segment (start 160.02 73.914) (end 155.956 73.914) (width 0.254) (layer F.Cu) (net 6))
 (segment (start 162.764 77.594) (end 164.084 78.914) (width 0.254) (layer F.Cu) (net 21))
 (segment (start 139.304 77.594) (end 162.764 77.594) (width 0.254) (layer F.Cu) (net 21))
 (segment (start 136.644 80.2531) (end 139.304 77.594) (width 0.254) (layer F.Cu) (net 21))
 (segment (start 125.233 80.2531) (end 136.644 80.2531) (width 0.254) (layer F.Cu) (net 21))
 (segment (start 122.911 82.5751) (end 125.233 80.2531) (width 0.254) (layer F.Cu) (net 21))
 (segment (start 121.666 82.5751) (end 122.911 82.5751) (width 0.254) (layer F.Cu) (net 21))
 (segment (start 121.666 83.566) (end 121.666 82.5751) (width 0.254) (layer F.Cu) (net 21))
 (segment (start 121.666 83.82) (end 121.666 83.566) (width 0.254) (layer F.Cu) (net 21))
 (segment (start 154.701 78.74) (end 151.892 78.74) (width 0.254) (layer F.Cu) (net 9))
 (segment (start 154.875 78.914) (end 154.701 78.74) (width 0.254) (layer F.Cu) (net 9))
 (segment (start 155.956 78.914) (end 154.875 78.914) (width 0.254) (layer F.Cu) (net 9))
 (segment (start 146.469 81.788) (end 145.288 81.788) (width 0.254) (layer F.Cu) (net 9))
 (segment (start 146.469 81.4187) (end 146.469 81.788) (width 0.254) (layer F.Cu) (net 9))
 (segment (start 147.281 80.6067) (end 146.469 81.4187) (width 0.254) (layer F.Cu) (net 9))
 (segment (start 149.168 80.6067) (end 147.281 80.6067) (width 0.254) (layer F.Cu) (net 9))
 (segment (start 150.811 78.964) (end 149.168 80.6067) (width 0.254) (layer F.Cu) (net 9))
 (segment (start 150.811 78.74) (end 150.811 78.964) (width 0.254) (layer F.Cu) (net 9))
 (segment (start 151.892 78.74) (end 150.811 78.74) (width 0.254) (layer F.Cu) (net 9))
 (segment (start 126.746 80.6575) (end 126.746 78.74) (width 0.254) (layer B.Cu) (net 11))
 (segment (start 122.288 85.1151) (end 126.746 80.6575) (width 0.254) (layer B.Cu) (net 11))
 (segment (start 121.666 85.1151) (end 122.288 85.1151) (width 0.254) (layer B.Cu) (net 11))
 (segment (start 121.666 86.106) (end 121.666 85.1151) (width 0.254) (layer B.Cu) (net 11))
 (segment (start 121.666 86.36) (end 121.666 86.106) (width 0.254) (layer B.Cu) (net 11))
 (segment (start 134.112 98.7407) (end 134.112 97.282) (width 0.254) (layer F.Cu) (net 18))
 (segment (start 133.858 98.9947) (end 134.112 98.7407) (width 0.254) (layer F.Cu) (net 18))
 (segment (start 133.858 100.076) (end 133.858 98.9947) (width 0.254) (layer F.Cu) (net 18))
 (segment (start 171.323 81.026) (end 172.72 81.026) (width 0.254) (layer B.Cu) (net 17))
 (segment (start 161.228 91.1207) (end 171.323 81.026) (width 0.254) (layer B.Cu) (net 17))
 (segment (start 160.782 91.1207) (end 161.228 91.1207) (width 0.254) (layer B.Cu) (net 17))
 (segment (start 160.782 92.202) (end 160.782 91.1207) (width 0.254) (layer B.Cu) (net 17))
 (segment (start 150.368 89.408) (end 147.828 89.408) (width 0.254) (layer F.Cu) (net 17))
 (segment (start 151.573 89.408) (end 150.368 89.408) (width 0.254) (layer B.Cu) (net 17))
 (segment (start 154.367 92.202) (end 151.573 89.408) (width 0.254) (layer B.Cu) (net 17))
 (segment (start 155.448 92.202) (end 154.367 92.202) (width 0.254) (layer B.Cu) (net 17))
 (segment (start 155.448 92.202) (end 160.782 92.202) (width 0.254) (layer F.Cu) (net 17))
 (segment (start 142.8 86.106) (end 172.72 86.106) (width 0.254) (layer F.Cu) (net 1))
 (segment (start 138.849 82.1551) (end 142.8 86.106) (width 0.254) (layer F.Cu) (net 1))
 (segment (start 138.849 81.788) (end 138.849 82.1551) (width 0.254) (layer F.Cu) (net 1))
 (segment (start 137.668 81.788) (end 138.849 81.788) (width 0.254) (layer F.Cu) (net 1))
 (segment (start 135.128 81.788) (end 137.668 81.788) (width 0.254) (layer F.Cu) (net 1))
 (segment (start 135.128 80.6067) (end 135.128 81.788) (width 0.254) (layer B.Cu) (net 1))
 (segment (start 135.913 79.8213) (end 135.128 80.6067) (width 0.254) (layer B.Cu) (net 1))
 (segment (start 136.144 79.8213) (end 135.913 79.8213) (width 0.254) (layer B.Cu) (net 1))
 (segment (start 136.144 78.74) (end 136.144 79.8213) (width 0.254) (layer B.Cu) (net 1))
 (segment (start 131.971 78.74) (end 136.144 78.74) (width 0.254) (layer F.Cu) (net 1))
 (segment (start 131.891 78.66) (end 131.971 78.74) (width 0.254) (layer F.Cu) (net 1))
 (segment (start 130.81 78.66) (end 131.891 78.66) (width 0.254) (layer F.Cu) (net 1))
 (segment (start 165.673 83.566) (end 172.72 83.566) (width 0.254) (layer F.Cu) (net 7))
 (segment (start 161.101 78.994) (end 165.673 83.566) (width 0.254) (layer F.Cu) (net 7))
 (segment (start 160.02 78.994) (end 161.101 78.994) (width 0.254) (layer F.Cu) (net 7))
 (segment (start 147.828 81.788) (end 150.368 81.788) (width 0.254) (layer F.Cu) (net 7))
 (segment (start 156.145 81.788) (end 150.368 81.788) (width 0.254) (layer F.Cu) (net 7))
 (segment (start 158.939 78.994) (end 156.145 81.788) (width 0.254) (layer F.Cu) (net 7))
 (segment (start 160.02 78.994) (end 158.939 78.994) (width 0.254) (layer F.Cu) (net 7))
 (segment (start 137.668 89.408) (end 135.128 89.408) (width 0.254) (layer F.Cu) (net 14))
 (segment (start 131.76 88.8316) (end 133.142 90.2132) (width 0.254) (layer B.Cu) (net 14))
 (segment (start 131.76 88.227) (end 131.76 88.8316) (width 0.254) (layer B.Cu) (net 14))
 (segment (start 136.398 83.5888) (end 131.76 88.227) (width 0.254) (layer B.Cu) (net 14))
 (segment (start 136.398 81.344) (end 136.398 83.5888) (width 0.254) (layer B.Cu) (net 14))
 (segment (start 140.107 77.6348) (end 136.398 81.344) (width 0.254) (layer B.Cu) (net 14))
 (segment (start 170.472 77.6348) (end 140.107 77.6348) (width 0.254) (layer B.Cu) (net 14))
 (segment (start 171.323 78.486) (end 170.472 77.6348) (width 0.254) (layer B.Cu) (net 14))
 (segment (start 172.72 78.486) (end 171.323 78.486) (width 0.254) (layer B.Cu) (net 14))
 (segment (start 133.947 89.408) (end 133.142 90.2132) (width 0.254) (layer B.Cu) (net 14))
 (segment (start 135.128 89.408) (end 133.947 89.408) (width 0.254) (layer B.Cu) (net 14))
 (segment (start 132.145 92.202) (end 131.064 92.202) (width 0.254) (layer B.Cu) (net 14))
 (segment (start 132.522 91.8249) (end 132.145 92.202) (width 0.254) (layer B.Cu) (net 14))
 (segment (start 132.522 90.8323) (end 132.522 91.8249) (width 0.254) (layer B.Cu) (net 14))
 (segment (start 133.142 90.2132) (end 132.522 90.8323) (width 0.254) (layer B.Cu) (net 14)))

